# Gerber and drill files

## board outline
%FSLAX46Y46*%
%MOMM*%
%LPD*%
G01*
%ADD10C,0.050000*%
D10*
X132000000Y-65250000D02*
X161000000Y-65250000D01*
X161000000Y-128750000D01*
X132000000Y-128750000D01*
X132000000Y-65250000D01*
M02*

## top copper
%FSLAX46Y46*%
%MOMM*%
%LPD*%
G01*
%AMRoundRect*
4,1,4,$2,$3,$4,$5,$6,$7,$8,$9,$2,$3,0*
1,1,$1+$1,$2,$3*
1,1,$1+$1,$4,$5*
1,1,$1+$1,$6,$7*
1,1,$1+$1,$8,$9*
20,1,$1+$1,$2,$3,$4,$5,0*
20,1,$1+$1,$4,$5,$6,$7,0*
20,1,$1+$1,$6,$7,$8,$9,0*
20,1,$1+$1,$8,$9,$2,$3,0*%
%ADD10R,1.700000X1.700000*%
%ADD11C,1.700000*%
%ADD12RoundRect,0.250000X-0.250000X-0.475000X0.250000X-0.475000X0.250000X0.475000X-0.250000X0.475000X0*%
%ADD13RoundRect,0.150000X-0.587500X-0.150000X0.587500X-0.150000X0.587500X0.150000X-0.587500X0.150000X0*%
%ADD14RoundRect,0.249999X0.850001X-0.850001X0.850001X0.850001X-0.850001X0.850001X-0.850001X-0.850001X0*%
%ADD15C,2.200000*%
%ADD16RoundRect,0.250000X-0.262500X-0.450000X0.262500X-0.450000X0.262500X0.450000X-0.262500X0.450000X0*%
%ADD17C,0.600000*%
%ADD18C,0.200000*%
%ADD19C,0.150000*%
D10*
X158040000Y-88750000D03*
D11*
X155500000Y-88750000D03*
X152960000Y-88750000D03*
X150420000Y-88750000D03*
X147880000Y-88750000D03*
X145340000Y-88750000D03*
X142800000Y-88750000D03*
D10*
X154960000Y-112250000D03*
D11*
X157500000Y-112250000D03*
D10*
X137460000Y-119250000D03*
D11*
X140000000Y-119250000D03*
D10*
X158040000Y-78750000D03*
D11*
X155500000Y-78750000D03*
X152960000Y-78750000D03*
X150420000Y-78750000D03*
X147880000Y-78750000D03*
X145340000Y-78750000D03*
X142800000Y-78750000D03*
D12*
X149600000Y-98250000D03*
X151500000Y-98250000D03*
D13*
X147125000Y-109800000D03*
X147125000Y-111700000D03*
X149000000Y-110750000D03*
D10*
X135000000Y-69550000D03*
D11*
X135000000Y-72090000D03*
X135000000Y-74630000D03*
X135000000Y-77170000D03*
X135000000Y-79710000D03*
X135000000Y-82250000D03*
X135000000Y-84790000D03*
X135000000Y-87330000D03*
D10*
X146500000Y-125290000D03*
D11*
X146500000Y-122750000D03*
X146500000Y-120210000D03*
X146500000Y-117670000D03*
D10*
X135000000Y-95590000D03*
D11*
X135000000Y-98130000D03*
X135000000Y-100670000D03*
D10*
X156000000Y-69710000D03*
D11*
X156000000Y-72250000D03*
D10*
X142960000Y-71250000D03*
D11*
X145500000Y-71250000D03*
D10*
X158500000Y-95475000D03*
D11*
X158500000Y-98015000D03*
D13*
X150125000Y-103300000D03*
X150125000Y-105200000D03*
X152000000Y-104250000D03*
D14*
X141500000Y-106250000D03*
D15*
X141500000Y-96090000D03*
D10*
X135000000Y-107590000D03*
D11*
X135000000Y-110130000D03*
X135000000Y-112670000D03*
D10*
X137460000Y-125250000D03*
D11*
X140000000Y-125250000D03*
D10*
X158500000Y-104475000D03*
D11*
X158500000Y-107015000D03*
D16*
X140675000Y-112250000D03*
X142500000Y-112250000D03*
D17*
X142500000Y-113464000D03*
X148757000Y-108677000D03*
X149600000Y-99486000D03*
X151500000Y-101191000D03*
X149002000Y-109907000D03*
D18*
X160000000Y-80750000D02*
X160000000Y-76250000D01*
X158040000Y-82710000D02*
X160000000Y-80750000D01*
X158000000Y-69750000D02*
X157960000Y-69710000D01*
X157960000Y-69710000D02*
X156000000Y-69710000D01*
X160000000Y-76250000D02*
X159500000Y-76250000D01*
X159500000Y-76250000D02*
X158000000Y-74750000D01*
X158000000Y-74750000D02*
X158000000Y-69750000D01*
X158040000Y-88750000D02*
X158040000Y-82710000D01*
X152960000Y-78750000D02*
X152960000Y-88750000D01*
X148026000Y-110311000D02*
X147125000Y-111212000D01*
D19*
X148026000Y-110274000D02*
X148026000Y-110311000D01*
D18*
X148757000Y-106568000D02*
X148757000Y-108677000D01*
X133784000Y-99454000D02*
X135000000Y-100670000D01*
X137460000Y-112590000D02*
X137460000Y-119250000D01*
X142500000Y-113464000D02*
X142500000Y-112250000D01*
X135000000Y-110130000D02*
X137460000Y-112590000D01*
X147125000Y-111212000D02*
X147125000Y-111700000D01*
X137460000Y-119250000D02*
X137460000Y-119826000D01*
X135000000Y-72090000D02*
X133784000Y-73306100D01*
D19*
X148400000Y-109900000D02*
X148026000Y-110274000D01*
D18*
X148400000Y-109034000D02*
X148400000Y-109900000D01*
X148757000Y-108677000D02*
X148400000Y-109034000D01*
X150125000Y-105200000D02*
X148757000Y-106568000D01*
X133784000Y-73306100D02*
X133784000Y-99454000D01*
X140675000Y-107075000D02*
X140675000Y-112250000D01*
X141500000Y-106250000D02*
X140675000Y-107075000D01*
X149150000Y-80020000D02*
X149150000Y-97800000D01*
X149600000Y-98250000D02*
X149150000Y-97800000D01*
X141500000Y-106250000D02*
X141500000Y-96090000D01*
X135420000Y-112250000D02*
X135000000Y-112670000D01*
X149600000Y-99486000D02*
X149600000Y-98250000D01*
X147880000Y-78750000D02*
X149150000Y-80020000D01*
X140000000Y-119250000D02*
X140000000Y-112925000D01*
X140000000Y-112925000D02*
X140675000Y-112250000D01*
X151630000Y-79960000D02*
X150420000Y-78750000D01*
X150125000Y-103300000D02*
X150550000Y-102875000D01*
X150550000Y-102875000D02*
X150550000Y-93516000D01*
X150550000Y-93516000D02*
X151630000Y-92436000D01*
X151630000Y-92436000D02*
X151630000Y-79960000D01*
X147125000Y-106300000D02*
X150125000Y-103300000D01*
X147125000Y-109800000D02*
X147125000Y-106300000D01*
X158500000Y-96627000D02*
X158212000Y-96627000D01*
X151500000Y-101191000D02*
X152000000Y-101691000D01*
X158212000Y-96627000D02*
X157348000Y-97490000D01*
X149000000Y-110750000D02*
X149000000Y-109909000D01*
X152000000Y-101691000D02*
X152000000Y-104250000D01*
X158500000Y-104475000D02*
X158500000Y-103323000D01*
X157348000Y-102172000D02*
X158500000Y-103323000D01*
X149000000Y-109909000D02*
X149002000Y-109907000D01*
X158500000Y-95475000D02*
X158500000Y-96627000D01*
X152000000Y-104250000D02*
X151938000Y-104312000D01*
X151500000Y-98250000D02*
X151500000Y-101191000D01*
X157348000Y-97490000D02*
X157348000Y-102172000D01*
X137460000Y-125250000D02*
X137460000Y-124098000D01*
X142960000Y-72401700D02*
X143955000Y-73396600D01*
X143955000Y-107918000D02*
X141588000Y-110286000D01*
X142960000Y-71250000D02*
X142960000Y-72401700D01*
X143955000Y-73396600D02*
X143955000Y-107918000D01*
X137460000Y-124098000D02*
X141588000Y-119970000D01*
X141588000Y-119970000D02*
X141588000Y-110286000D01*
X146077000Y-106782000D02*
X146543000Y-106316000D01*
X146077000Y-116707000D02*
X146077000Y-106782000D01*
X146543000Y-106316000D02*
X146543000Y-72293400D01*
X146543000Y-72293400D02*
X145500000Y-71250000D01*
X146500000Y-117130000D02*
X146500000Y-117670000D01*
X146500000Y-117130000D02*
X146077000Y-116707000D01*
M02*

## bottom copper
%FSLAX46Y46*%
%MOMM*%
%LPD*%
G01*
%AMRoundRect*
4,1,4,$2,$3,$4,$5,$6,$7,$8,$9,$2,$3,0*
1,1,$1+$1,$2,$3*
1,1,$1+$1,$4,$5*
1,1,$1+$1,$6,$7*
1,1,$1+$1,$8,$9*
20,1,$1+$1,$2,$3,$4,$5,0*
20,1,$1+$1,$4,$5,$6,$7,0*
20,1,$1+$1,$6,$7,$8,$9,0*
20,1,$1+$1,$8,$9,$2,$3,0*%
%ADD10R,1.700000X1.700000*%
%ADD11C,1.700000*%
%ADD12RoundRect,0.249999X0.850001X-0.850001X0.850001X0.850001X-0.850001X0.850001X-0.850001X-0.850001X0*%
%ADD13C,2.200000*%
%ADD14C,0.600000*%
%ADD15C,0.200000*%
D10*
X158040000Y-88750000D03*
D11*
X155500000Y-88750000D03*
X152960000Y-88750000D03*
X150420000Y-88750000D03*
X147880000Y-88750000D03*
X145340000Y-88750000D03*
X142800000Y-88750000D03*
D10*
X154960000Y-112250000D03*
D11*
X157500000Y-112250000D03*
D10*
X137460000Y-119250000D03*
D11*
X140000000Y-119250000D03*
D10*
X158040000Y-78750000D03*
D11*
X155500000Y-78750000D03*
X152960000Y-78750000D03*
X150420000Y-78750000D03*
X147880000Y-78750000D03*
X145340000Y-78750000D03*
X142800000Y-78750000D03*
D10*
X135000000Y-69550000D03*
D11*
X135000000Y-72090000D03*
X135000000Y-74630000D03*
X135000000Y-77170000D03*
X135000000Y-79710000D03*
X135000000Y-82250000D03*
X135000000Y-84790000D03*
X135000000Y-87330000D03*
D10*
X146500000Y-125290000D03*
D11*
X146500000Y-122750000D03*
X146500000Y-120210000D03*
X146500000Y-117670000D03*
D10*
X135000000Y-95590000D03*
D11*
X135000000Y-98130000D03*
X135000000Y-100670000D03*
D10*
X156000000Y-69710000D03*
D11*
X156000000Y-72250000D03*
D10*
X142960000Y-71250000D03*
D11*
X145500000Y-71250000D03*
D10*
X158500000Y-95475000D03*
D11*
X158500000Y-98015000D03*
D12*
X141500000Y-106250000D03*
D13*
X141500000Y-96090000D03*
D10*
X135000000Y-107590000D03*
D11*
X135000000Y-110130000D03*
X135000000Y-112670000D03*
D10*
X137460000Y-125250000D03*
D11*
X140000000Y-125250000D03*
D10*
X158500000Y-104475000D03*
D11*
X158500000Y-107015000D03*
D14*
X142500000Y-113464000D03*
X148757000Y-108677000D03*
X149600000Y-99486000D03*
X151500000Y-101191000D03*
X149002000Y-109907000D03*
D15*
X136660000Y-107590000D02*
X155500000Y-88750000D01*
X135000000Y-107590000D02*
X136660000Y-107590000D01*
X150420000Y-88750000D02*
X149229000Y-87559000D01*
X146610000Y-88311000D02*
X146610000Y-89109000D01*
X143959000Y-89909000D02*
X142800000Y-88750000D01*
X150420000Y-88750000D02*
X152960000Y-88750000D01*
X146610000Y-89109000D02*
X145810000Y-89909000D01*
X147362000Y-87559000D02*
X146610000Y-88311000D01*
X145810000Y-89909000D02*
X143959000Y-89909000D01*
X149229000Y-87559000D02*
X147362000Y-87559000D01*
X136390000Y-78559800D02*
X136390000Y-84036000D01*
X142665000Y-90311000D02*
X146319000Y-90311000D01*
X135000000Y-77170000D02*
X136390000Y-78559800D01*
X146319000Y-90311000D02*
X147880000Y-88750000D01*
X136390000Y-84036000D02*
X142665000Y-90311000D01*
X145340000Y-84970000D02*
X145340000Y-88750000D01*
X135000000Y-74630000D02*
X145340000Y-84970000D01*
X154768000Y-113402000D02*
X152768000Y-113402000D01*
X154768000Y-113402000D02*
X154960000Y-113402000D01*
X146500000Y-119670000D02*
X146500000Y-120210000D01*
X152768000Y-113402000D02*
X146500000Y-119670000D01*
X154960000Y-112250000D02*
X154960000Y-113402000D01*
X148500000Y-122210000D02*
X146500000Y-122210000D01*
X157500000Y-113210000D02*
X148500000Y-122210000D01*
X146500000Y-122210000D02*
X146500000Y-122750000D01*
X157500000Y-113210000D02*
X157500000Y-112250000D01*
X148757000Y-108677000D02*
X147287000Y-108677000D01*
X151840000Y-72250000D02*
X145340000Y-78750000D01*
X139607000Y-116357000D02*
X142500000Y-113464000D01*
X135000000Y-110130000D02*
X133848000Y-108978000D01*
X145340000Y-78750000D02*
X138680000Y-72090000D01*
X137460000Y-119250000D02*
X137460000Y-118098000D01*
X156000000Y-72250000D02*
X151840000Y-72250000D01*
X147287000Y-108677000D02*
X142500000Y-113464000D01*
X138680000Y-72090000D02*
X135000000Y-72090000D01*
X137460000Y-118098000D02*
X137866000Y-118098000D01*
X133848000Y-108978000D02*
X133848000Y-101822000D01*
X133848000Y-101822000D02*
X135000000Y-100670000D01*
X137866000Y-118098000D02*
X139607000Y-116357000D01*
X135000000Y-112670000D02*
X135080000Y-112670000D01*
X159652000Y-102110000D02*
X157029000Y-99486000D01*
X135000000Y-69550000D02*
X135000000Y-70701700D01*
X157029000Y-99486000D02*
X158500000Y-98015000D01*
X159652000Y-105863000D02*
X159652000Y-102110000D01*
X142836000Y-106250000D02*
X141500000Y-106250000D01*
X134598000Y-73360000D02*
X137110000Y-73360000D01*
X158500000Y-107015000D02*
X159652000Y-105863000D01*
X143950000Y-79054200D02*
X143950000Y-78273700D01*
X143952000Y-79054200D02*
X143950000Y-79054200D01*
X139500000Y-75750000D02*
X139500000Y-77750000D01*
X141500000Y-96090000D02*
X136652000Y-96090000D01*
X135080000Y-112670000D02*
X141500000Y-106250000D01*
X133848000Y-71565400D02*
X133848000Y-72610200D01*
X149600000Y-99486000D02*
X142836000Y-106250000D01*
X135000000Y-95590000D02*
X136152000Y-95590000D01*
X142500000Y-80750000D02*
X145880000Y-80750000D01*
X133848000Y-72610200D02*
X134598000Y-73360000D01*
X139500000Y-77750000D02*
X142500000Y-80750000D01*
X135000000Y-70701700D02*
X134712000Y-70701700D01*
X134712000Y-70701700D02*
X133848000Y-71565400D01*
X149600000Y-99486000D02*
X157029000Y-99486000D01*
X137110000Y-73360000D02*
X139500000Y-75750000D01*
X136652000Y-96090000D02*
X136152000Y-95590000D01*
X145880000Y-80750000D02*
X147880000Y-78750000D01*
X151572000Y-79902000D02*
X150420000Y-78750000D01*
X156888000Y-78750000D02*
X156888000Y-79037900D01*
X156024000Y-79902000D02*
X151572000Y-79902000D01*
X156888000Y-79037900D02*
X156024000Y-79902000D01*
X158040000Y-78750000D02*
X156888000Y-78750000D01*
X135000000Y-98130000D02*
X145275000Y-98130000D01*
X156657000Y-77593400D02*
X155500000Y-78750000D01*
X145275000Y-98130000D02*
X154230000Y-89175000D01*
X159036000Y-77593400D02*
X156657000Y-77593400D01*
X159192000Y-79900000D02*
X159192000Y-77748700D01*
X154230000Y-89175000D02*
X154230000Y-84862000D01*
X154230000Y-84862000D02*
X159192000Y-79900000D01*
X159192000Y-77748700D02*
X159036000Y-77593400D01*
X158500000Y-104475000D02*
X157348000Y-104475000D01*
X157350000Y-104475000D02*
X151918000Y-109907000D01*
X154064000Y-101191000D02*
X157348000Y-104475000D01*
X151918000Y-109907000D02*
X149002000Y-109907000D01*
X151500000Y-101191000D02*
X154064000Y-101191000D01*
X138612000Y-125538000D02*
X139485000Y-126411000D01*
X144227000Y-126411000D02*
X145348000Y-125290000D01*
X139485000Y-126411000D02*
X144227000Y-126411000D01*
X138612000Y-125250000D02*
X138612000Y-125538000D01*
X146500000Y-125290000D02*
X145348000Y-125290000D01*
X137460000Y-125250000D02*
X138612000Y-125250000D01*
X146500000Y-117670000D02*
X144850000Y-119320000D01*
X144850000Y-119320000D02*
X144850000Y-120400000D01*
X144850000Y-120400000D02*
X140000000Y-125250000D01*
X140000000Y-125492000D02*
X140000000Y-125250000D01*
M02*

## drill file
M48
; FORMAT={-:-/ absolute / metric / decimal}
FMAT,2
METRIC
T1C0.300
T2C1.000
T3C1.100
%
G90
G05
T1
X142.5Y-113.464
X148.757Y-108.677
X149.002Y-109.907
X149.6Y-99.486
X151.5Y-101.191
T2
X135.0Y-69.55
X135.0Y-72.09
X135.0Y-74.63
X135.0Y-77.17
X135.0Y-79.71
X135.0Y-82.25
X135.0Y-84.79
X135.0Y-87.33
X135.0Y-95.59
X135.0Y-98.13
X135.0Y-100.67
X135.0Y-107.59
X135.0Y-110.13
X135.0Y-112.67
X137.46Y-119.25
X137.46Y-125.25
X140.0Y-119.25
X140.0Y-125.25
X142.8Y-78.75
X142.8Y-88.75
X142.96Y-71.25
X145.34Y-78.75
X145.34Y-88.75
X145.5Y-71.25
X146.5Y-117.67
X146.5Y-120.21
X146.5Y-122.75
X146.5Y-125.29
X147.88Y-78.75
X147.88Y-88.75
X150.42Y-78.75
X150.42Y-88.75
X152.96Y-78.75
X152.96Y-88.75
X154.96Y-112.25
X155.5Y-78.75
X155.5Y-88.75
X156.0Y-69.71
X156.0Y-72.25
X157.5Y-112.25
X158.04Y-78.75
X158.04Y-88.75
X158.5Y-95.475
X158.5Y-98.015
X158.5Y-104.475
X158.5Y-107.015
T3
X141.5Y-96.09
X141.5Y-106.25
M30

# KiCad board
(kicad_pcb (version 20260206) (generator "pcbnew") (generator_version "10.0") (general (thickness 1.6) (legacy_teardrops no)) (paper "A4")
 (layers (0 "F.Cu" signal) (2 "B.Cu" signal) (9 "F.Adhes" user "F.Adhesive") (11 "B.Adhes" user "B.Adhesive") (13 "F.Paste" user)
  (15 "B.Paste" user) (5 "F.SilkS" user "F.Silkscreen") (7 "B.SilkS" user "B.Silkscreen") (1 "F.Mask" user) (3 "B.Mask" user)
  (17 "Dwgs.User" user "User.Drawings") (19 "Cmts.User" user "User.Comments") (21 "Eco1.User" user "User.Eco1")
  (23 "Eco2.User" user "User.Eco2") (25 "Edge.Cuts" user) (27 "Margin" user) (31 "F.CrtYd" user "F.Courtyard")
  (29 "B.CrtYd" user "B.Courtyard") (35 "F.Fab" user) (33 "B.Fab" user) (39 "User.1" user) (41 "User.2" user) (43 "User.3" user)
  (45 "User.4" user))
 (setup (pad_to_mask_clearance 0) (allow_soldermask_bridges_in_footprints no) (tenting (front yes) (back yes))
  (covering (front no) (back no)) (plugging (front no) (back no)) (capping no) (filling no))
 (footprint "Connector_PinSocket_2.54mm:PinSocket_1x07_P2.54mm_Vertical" (layer "F.Cu") (at 158.04 88.75 -90)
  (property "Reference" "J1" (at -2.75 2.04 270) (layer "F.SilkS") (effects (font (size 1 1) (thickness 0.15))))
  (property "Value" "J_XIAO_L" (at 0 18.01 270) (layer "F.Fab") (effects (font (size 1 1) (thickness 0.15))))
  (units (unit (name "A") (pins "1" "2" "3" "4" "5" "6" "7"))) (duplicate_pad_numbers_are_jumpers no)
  (pad "1" thru_hole rect (at 0 0 270) (size 1.7 1.7) (drill 1) (layers "*.Cu" "*.Mask") (remove_unused_layers no) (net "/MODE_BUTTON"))
  (pad "2" thru_hole circle (at 0 2.54 270) (size 1.7 1.7) (drill 1) (layers "*.Cu" "*.Mask") (remove_unused_layers no) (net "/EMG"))
  (pad "3" thru_hole circle (at 0 5.08 270) (size 1.7 1.7) (drill 1) (layers "*.Cu" "*.Mask") (remove_unused_layers no) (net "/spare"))
  (pad "4" thru_hole circle (at 0 7.62 270) (size 1.7 1.7) (drill 1) (layers "*.Cu" "*.Mask") (remove_unused_layers no) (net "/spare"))
  (pad "5" thru_hole circle (at 0 10.16 270) (size 1.7 1.7) (drill 1) (layers "*.Cu" "*.Mask") (remove_unused_layers no) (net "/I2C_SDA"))
  (pad "6" thru_hole circle (at 0 12.7 270) (size 1.7 1.7) (drill 1) (layers "*.Cu" "*.Mask") (remove_unused_layers no) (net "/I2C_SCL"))
  (pad "7" thru_hole circle (at 0 15.24 270) (size 1.7 1.7) (drill 1) (layers "*.Cu" "*.Mask") (remove_unused_layers no) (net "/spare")))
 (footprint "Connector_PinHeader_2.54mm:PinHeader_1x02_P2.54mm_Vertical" (layer "F.Cu") (at 154.96 112.25 90)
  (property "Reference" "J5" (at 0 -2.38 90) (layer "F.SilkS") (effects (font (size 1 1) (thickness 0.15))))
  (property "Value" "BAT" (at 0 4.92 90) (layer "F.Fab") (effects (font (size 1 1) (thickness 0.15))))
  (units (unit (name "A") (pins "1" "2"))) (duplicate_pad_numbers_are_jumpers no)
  (pad "1" thru_hole rect (at 0 0 90) (size 1.7 1.7) (drill 1) (layers "*.Cu" "*.Mask") (remove_unused_layers no) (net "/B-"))
  (pad "2" thru_hole circle (at 0 2.54 90) (size 1.7 1.7) (drill 1) (layers "*.Cu" "*.Mask") (remove_unused_layers no) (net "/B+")))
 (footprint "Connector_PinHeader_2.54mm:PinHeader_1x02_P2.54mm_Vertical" (layer "F.Cu") (at 137.46 119.25 90)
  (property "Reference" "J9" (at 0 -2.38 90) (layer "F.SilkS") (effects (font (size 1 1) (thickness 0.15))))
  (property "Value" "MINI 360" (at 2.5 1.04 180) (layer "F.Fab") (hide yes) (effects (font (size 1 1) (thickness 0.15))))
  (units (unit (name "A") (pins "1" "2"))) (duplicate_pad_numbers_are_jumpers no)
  (pad "1" thru_hole rect (at 0 0 90) (size 1.7 1.7) (drill 1) (layers "*.Cu" "*.Mask") (remove_unused_layers no) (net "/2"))
  (pad "2" thru_hole circle (at 0 2.54 90) (size 1.7 1.7) (drill 1) (layers "*.Cu" "*.Mask") (remove_unused_layers no) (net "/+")))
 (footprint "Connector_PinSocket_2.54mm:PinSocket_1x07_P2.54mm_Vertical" (layer "F.Cu") (at 158.04 78.75 -90)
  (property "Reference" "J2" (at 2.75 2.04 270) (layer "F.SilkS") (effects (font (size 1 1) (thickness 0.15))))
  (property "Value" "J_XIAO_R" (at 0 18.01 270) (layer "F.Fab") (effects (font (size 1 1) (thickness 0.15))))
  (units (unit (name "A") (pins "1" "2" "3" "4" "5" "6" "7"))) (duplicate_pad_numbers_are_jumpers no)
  (pad "1" thru_hole rect (at 0 0 270) (size 1.7 1.7) (drill 1) (layers "*.Cu" "*.Mask") (remove_unused_layers no) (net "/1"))
  (pad "2" thru_hole circle (at 0 2.54 270) (size 1.7 1.7) (drill 1) (layers "*.Cu" "*.Mask") (remove_unused_layers no) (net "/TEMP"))
  (pad "3" thru_hole circle (at 0 5.08 270) (size 1.7 1.7) (drill 1) (layers "*.Cu" "*.Mask") (remove_unused_layers no) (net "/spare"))
  (pad "4" thru_hole circle (at 0 7.62 270) (size 1.7 1.7) (drill 1) (layers "*.Cu" "*.Mask") (remove_unused_layers no) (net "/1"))
  (pad "5" thru_hole circle (at 0 10.16 270) (size 1.7 1.7) (drill 1) (layers "*.Cu" "*.Mask") (remove_unused_layers no) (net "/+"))
  (pad "6" thru_hole circle (at 0 12.7 270) (size 1.7 1.7) (drill 1) (layers "*.Cu" "*.Mask") (remove_unused_layers no) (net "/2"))
  (pad "7" thru_hole circle (at 0 15.24 270) (size 1.7 1.7) (drill 1) (layers "*.Cu" "*.Mask") (remove_unused_layers no) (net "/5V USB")))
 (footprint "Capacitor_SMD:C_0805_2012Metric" (layer "F.Cu") (at 150.55 98.25)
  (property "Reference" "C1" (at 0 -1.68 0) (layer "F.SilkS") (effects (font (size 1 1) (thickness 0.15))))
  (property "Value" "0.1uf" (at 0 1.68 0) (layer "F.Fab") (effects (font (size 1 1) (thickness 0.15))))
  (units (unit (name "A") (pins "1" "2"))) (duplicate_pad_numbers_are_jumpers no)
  (pad "1" smd roundrect (at -0.95 0) (size 1 1.45) (layers "F.Cu" "F.Mask" "F.Paste") (roundrect_rratio 0.25) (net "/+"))
  (pad "2" smd roundrect (at 0.95 0) (size 1 1.45) (layers "F.Cu" "F.Mask" "F.Paste") (roundrect_rratio 0.25) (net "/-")))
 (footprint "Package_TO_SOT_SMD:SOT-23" (layer "F.Cu") (at 148.0625 110.75)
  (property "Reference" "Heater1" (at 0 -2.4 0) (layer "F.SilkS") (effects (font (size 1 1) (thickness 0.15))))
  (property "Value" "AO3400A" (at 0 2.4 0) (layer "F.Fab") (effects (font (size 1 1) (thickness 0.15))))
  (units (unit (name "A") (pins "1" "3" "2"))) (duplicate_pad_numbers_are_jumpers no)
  (pad "1" smd roundrect (at -0.9375 -0.95) (size 1.475 0.6) (layers "F.Cu" "F.Mask" "F.Paste") (roundrect_rratio 0.25) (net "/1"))
  (pad "2" smd roundrect (at -0.9375 0.95) (size 1.475 0.6) (layers "F.Cu" "F.Mask" "F.Paste") (roundrect_rratio 0.25) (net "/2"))
  (pad "3" smd roundrect (at 0.9375 0) (size 1.475 0.6) (layers "F.Cu" "F.Mask" "F.Paste") (roundrect_rratio 0.25) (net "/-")))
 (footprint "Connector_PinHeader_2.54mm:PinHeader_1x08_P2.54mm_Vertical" (layer "F.Cu") (at 135 69.55)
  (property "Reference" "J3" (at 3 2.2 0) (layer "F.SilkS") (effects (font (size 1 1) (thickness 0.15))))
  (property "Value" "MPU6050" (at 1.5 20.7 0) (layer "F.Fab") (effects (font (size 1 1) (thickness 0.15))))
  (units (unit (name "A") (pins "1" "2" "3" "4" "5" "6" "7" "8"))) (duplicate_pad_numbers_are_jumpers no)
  (pad "1" thru_hole rect (at 0 0) (size 1.7 1.7) (drill 1) (layers "*.Cu" "*.Mask") (remove_unused_layers no) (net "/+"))
  (pad "2" thru_hole circle (at 0 2.54) (size 1.7 1.7) (drill 1) (layers "*.Cu" "*.Mask") (remove_unused_layers no) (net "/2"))
  (pad "3" thru_hole circle (at 0 5.08) (size 1.7 1.7) (drill 1) (layers "*.Cu" "*.Mask") (remove_unused_layers no) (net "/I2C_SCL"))
  (pad "4" thru_hole circle (at 0 7.62) (size 1.7 1.7) (drill 1) (layers "*.Cu" "*.Mask") (remove_unused_layers no) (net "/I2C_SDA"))
  (pad "5" thru_hole circle (at 0 10.16) (size 1.7 1.7) (drill 1) (layers "*.Cu" "*.Mask") (remove_unused_layers no) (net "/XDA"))
  (pad "6" thru_hole circle (at 0 12.7) (size 1.7 1.7) (drill 1) (layers "*.Cu" "*.Mask") (remove_unused_layers no) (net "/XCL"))
  (pad "7" thru_hole circle (at 0 15.24) (size 1.7 1.7) (drill 1) (layers "*.Cu" "*.Mask") (remove_unused_layers no) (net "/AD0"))
  (pad "8" thru_hole circle (at 0 17.78) (size 1.7 1.7) (drill 1) (layers "*.Cu" "*.Mask") (remove_unused_layers no) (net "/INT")))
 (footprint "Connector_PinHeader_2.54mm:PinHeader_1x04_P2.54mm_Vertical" (layer "F.Cu") (at 146.5 125.29 180)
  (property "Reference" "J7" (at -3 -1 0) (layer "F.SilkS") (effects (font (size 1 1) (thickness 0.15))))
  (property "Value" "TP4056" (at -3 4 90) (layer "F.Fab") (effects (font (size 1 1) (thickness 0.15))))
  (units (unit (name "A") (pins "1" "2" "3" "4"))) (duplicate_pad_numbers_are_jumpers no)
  (pad "1" thru_hole rect (at 0 0 180) (size 1.7 1.7) (drill 1) (layers "*.Cu" "*.Mask") (remove_unused_layers no) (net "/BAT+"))
  (pad "2" thru_hole circle (at 0 2.54 180) (size 1.7 1.7) (drill 1) (layers "*.Cu" "*.Mask") (remove_unused_layers no) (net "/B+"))
  (pad "3" thru_hole circle (at 0 5.08 180) (size 1.7 1.7) (drill 1) (layers "*.Cu" "*.Mask") (remove_unused_layers no) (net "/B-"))
  (pad "4" thru_hole circle (at 0 7.62 180) (size 1.7 1.7) (drill 1) (layers "*.Cu" "*.Mask") (remove_unused_layers no) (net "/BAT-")))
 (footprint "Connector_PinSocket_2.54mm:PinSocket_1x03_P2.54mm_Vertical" (layer "F.Cu") (at 135 95.59)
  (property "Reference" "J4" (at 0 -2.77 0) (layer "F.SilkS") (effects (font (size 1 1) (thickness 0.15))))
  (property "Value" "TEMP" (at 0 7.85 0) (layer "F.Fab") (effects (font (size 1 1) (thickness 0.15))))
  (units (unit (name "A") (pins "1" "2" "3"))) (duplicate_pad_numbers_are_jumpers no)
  (pad "1" thru_hole rect (at 0 0) (size 1.7 1.7) (drill 1) (layers "*.Cu" "*.Mask") (remove_unused_layers no) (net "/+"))
  (pad "2" thru_hole circle (at 0 2.54) (size 1.7 1.7) (drill 1) (layers "*.Cu" "*.Mask") (remove_unused_layers no) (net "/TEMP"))
  (pad "3" thru_hole circle (at 0 5.08) (size 1.7 1.7) (drill 1) (layers "*.Cu" "*.Mask") (remove_unused_layers no) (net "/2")))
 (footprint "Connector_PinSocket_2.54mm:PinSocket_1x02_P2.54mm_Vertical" (layer "F.Cu") (at 156 69.71)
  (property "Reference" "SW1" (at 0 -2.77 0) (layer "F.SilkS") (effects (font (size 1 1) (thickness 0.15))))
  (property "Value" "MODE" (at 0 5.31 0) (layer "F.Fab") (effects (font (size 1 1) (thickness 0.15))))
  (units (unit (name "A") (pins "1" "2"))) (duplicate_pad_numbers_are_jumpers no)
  (pad "1" thru_hole rect (at 0 0) (size 1.7 1.7) (drill 1) (layers "*.Cu" "*.Mask") (remove_unused_layers no) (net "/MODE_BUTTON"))
  (pad "2" thru_hole circle (at 0 2.54) (size 1.7 1.7) (drill 1) (layers "*.Cu" "*.Mask") (remove_unused_layers no) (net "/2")))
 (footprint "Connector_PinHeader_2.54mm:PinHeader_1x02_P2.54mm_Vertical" (layer "F.Cu") (at 142.96 71.25 90)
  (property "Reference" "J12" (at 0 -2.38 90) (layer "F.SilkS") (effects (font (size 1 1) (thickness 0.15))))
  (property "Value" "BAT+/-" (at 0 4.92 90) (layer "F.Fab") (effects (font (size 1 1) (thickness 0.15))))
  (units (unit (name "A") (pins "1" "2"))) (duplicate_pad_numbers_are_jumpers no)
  (pad "1" thru_hole rect (at 0 0 90) (size 1.7 1.7) (drill 1) (layers "*.Cu" "*.Mask") (remove_unused_layers no) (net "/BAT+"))
  (pad "2" thru_hole circle (at 0 2.54 90) (size 1.7 1.7) (drill 1) (layers "*.Cu" "*.Mask") (remove_unused_layers no) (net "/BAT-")))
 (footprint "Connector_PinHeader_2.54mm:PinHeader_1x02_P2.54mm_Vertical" (layer "F.Cu") (at 158.5 95.475)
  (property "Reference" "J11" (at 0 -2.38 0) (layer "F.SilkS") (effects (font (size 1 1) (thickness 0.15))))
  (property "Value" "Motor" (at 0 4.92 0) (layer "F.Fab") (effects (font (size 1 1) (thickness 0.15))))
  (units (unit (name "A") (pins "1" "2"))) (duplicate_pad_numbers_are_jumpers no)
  (pad "1" thru_hole rect (at 0 0) (size 1.7 1.7) (drill 1) (layers "*.Cu" "*.Mask") (remove_unused_layers no) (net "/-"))
  (pad "2" thru_hole circle (at 0 2.54) (size 1.7 1.7) (drill 1) (layers "*.Cu" "*.Mask") (remove_unused_layers no) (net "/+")))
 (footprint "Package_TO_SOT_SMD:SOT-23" (layer "F.Cu") (at 151.0625 104.25)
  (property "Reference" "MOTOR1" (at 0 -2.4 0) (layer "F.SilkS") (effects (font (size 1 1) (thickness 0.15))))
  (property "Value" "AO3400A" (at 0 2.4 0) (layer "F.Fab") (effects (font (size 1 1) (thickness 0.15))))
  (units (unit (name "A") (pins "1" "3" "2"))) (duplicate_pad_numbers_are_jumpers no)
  (pad "1" smd roundrect (at -0.9375 -0.95) (size 1.475 0.6) (layers "F.Cu" "F.Mask" "F.Paste") (roundrect_rratio 0.25) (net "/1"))
  (pad "2" smd roundrect (at -0.9375 0.95) (size 1.475 0.6) (layers "F.Cu" "F.Mask" "F.Paste") (roundrect_rratio 0.25) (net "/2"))
  (pad "3" smd roundrect (at 0.9375 0) (size 1.475 0.6) (layers "F.Cu" "F.Mask" "F.Paste") (roundrect_rratio 0.25) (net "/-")))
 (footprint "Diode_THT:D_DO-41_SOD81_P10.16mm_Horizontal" (layer "F.Cu") (at 141.5 106.25 90)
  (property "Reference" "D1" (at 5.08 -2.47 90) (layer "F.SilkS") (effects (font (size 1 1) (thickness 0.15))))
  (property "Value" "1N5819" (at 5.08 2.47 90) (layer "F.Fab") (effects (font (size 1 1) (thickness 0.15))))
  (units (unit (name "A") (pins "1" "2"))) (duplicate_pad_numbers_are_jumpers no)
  (pad "1" thru_hole roundrect (at 0 0 90) (size 2.2 2.2) (drill 1.1) (layers "*.Cu" "*.Mask") (remove_unused_layers no)
   (roundrect_rratio 0.113636) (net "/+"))
  (pad "2" thru_hole circle (at 10.16 0 90) (size 2.2 2.2) (drill 1.1) (layers "*.Cu" "*.Mask") (remove_unused_layers no) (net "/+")))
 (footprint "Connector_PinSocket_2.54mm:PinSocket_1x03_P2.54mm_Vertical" (layer "F.Cu") (at 135 107.59)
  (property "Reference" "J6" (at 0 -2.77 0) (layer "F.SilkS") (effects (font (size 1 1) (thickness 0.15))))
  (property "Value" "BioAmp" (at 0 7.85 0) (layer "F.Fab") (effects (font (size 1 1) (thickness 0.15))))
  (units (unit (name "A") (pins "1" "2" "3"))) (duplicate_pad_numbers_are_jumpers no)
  (pad "1" thru_hole rect (at 0 0) (size 1.7 1.7) (drill 1) (layers "*.Cu" "*.Mask") (remove_unused_layers no) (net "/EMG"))
  (pad "2" thru_hole circle (at 0 2.54) (size 1.7 1.7) (drill 1) (layers "*.Cu" "*.Mask") (remove_unused_layers no) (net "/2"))
  (pad "3" thru_hole circle (at 0 5.08) (size 1.7 1.7) (drill 1) (layers "*.Cu" "*.Mask") (remove_unused_layers no) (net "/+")))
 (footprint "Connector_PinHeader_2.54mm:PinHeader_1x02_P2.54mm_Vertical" (layer "F.Cu") (at 137.46 125.25 90)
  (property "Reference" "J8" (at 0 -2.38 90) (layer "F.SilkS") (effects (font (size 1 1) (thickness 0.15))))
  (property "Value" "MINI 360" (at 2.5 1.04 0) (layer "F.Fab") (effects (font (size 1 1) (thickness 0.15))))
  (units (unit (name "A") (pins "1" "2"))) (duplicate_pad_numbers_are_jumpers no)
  (pad "1" thru_hole rect (at 0 0 90) (size 1.7 1.7) (drill 1) (layers "*.Cu" "*.Mask") (remove_unused_layers no) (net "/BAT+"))
  (pad "2" thru_hole circle (at 0 2.54 90) (size 1.7 1.7) (drill 1) (layers "*.Cu" "*.Mask") (remove_unused_layers no) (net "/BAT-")))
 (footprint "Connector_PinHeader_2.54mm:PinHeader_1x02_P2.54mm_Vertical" (layer "F.Cu") (at 158.5 104.475)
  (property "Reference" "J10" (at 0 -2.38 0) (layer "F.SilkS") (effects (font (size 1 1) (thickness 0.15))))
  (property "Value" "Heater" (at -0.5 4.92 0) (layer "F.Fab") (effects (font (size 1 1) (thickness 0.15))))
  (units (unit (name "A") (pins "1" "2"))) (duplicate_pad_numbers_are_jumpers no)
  (pad "1" thru_hole rect (at 0 0) (size 1.7 1.7) (drill 1) (layers "*.Cu" "*.Mask") (remove_unused_layers no) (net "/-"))
  (pad "2" thru_hole circle (at 0 2.54) (size 1.7 1.7) (drill 1) (layers "*.Cu" "*.Mask") (remove_unused_layers no) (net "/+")))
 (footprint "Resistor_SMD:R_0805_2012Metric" (layer "F.Cu") (at 141.5875 112.25)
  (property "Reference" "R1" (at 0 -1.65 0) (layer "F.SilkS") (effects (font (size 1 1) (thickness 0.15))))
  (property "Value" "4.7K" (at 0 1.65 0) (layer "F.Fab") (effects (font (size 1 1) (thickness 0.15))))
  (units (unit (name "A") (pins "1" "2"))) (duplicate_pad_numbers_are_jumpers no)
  (pad "1" smd roundrect (at -0.9125 0) (size 1.025 1.4) (layers "F.Cu" "F.Mask" "F.Paste") (roundrect_rratio 0.243902) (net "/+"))
  (pad "2" smd roundrect (at 0.9125 0) (size 1.025 1.4) (layers "F.Cu" "F.Mask" "F.Paste") (roundrect_rratio 0.243902) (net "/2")))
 (gr_rect (start 132 65.25) (end 161 128.75) (stroke (width 0.05) (type default)) (fill no) (layer "Edge.Cuts"))
 (segment (start 160 80.75) (end 160 76.25) (width 0.2) (layer "F.Cu") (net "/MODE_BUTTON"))
 (segment (start 158.04 82.71) (end 160 80.75) (width 0.2) (layer "F.Cu") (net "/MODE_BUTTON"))
 (segment (start 158 69.75) (end 157.96 69.71) (width 0.2) (layer "F.Cu") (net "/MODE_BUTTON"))
 (segment (start 157.96 69.71) (end 156 69.71) (width 0.2) (layer "F.Cu") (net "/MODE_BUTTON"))
 (segment (start 160 76.25) (end 159.5 76.25) (width 0.2) (layer "F.Cu") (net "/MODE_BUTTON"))
 (segment (start 159.5 76.25) (end 158 74.75) (width 0.2) (layer "F.Cu") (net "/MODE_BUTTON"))
 (segment (start 158 74.75) (end 158 69.75) (width 0.2) (layer "F.Cu") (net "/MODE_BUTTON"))
 (segment (start 158.04 88.75) (end 158.04 82.71) (width 0.2) (layer "F.Cu") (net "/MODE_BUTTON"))
 (segment (start 136.66 107.59) (end 155.5 88.75) (width 0.2) (layer "B.Cu") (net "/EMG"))
 (segment (start 135 107.59) (end 136.66 107.59) (width 0.2) (layer "B.Cu") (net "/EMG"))
 (segment (start 152.96 78.75) (end 152.96 88.75) (width 0.2) (layer "F.Cu") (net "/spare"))
 (segment (start 150.42 88.75) (end 149.229 87.559) (width 0.2) (layer "B.Cu") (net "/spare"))
 (segment (start 146.61 88.311) (end 146.61 89.109) (width 0.2) (layer "B.Cu") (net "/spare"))
 (segment (start 143.959 89.909) (end 142.8 88.75) (width 0.2) (layer "B.Cu") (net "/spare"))
 (segment (start 150.42 88.75) (end 152.96 88.75) (width 0.2) (layer "B.Cu") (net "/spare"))
 (segment (start 146.61 89.109) (end 145.81 89.909) (width 0.2) (layer "B.Cu") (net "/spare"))
 (segment (start 147.362 87.559) (end 146.61 88.311) (width 0.2) (layer "B.Cu") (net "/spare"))
 (segment (start 145.81 89.909) (end 143.959 89.909) (width 0.2) (layer "B.Cu") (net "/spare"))
 (segment (start 149.229 87.559) (end 147.362 87.559) (width 0.2) (layer "B.Cu") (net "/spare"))
 (segment (start 136.39 78.5598) (end 136.39 84.036) (width 0.2) (layer "B.Cu") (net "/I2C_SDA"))
 (segment (start 142.665 90.311) (end 146.319 90.311) (width 0.2) (layer "B.Cu") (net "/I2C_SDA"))
 (segment (start 135 77.17) (end 136.39 78.5598) (width 0.2) (layer "B.Cu") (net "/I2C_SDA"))
 (segment (start 146.319 90.311) (end 147.88 88.75) (width 0.2) (layer "B.Cu") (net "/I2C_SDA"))
 (segment (start 136.39 84.036) (end 142.665 90.311) (width 0.2) (layer "B.Cu") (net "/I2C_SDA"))
 (segment (start 145.34 84.97) (end 145.34 88.75) (width 0.2) (layer "B.Cu") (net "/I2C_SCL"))
 (segment (start 135 74.63) (end 145.34 84.97) (width 0.2) (layer "B.Cu") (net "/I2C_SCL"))
 (segment (start 154.768 113.402) (end 152.768 113.402) (width 0.2) (layer "B.Cu") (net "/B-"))
 (segment (start 154.768 113.402) (end 154.96 113.402) (width 0.2) (layer "B.Cu") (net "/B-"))
 (segment (start 146.5 119.67) (end 146.5 120.21) (width 0.2) (layer "B.Cu") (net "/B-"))
 (segment (start 152.768 113.402) (end 146.5 119.67) (width 0.2) (layer "B.Cu") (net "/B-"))
 (segment (start 154.96 112.25) (end 154.96 113.402) (width 0.2) (layer "B.Cu") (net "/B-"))
 (segment (start 148.5 122.21) (end 146.5 122.21) (width 0.2) (layer "B.Cu") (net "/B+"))
 (segment (start 157.5 113.21) (end 148.5 122.21) (width 0.2) (layer "B.Cu") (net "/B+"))
 (segment (start 146.5 122.21) (end 146.5 122.75) (width 0.2) (layer "B.Cu") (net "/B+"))
 (segment (start 157.5 113.21) (end 157.5 112.25) (width 0.2) (layer "B.Cu") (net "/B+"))
 (segment (start 148.026 110.311) (end 147.125 111.212) (width 0.2) (layer "F.Cu") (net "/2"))
 (segment (start 148.026 110.274) (end 148.026 110.311) (width 0.15) (layer "F.Cu") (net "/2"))
 (segment (start 148.757 106.568) (end 148.757 108.677) (width 0.2) (layer "F.Cu") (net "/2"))
 (segment (start 133.784 99.454) (end 135 100.67) (width 0.2) (layer "F.Cu") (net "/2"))
 (segment (start 137.46 112.59) (end 137.46 119.25) (width 0.2) (layer "F.Cu") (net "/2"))
 (segment (start 142.5 113.464) (end 142.5 112.25) (width 0.2) (layer "F.Cu") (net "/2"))
 (segment (start 135 110.13) (end 137.46 112.59) (width 0.2) (layer "F.Cu") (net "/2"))
 (segment (start 147.125 111.212) (end 147.125 111.7) (width 0.2) (layer "F.Cu") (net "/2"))
 (segment (start 137.46 119.25) (end 137.46 119.826) (width 0.2) (layer "F.Cu") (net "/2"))
 (segment (start 135 72.09) (end 133.784 73.3061) (width 0.2) (layer "F.Cu") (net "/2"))
 (segment (start 148.4 109.9) (end 148.026 110.274) (width 0.15) (layer "F.Cu") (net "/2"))
 (segment (start 148.4 109.034) (end 148.4 109.9) (width 0.2) (layer "F.Cu") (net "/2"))
 (segment (start 148.757 108.677) (end 148.4 109.034) (width 0.2) (layer "F.Cu") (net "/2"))
 (segment (start 150.125 105.2) (end 148.757 106.568) (width 0.2) (layer "F.Cu") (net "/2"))
 (segment (start 133.784 73.3061) (end 133.784 99.454) (width 0.2) (layer "F.Cu") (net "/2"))
 (via (at 142.5 113.464) (size 0.6) (drill 0.3) (layers "F.Cu" "B.Cu") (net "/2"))
 (via (at 148.757 108.677) (size 0.6) (drill 0.3) (layers "F.Cu" "B.Cu") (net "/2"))
 (segment (start 148.757 108.677) (end 147.287 108.677) (width 0.2) (layer "B.Cu") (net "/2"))
 (segment (start 151.84 72.25) (end 145.34 78.75) (width 0.2) (layer "B.Cu") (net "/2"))
 (segment (start 139.607 116.357) (end 142.5 113.464) (width 0.2) (layer "B.Cu") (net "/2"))
 (segment (start 135 110.13) (end 133.848 108.978) (width 0.2) (layer "B.Cu") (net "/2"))
 (segment (start 145.34 78.75) (end 138.68 72.09) (width 0.2) (layer "B.Cu") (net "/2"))
 (segment (start 137.46 119.25) (end 137.46 118.098) (width 0.2) (layer "B.Cu") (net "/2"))
 (segment (start 156 72.25) (end 151.84 72.25) (width 0.2) (layer "B.Cu") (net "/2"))
 (segment (start 147.287 108.677) (end 142.5 113.464) (width 0.2) (layer "B.Cu") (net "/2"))
 (segment (start 138.68 72.09) (end 135 72.09) (width 0.2) (layer "B.Cu") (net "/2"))
 (segment (start 137.46 118.098) (end 137.866 118.098) (width 0.2) (layer "B.Cu") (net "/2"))
 (segment (start 133.848 108.978) (end 133.848 101.822) (width 0.2) (layer "B.Cu") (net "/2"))
 (segment (start 133.848 101.822) (end 135 100.67) (width 0.2) (layer "B.Cu") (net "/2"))
 (segment (start 137.866 118.098) (end 139.607 116.357) (width 0.2) (layer "B.Cu") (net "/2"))
 (segment (start 140.675 107.075) (end 140.675 112.25) (width 0.2) (layer "F.Cu") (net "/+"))
 (segment (start 141.5 106.25) (end 140.675 107.075) (width 0.2) (layer "F.Cu") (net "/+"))
 (segment (start 149.15 80.02) (end 149.15 97.8) (width 0.2) (layer "F.Cu") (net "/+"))
 (segment (start 149.6 98.25) (end 149.15 97.8) (width 0.2) (layer "F.Cu") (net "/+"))
 (segment (start 141.5 106.25) (end 141.5 96.09) (width 0.2) (layer "F.Cu") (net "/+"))
 (segment (start 135.42 112.25) (end 135 112.67) (width 0.2) (layer "F.Cu") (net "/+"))
 (segment (start 149.6 99.486) (end 149.6 98.25) (width 0.2) (layer "F.Cu") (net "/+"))
 (segment (start 147.88 78.75) (end 149.15 80.02) (width 0.2) (layer "F.Cu") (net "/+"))
 (segment (start 140 119.25) (end 140 112.925) (width 0.2) (layer "F.Cu") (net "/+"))
 (segment (start 140 112.925) (end 140.675 112.25) (width 0.2) (layer "F.Cu") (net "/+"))
 (via (at 149.6 99.486) (size 0.6) (drill 0.3) (layers "F.Cu" "B.Cu") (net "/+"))
 (segment (start 135 112.67) (end 135.08 112.67) (width 0.2) (layer "B.Cu") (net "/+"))
 (segment (start 159.652 102.11) (end 157.029 99.486) (width 0.2) (layer "B.Cu") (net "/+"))
 (segment (start 135 69.55) (end 135 70.7017) (width 0.2) (layer "B.Cu") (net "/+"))
 (segment (start 157.029 99.486) (end 158.5 98.015) (width 0.2) (layer "B.Cu") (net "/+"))
 (segment (start 159.652 105.863) (end 159.652 102.11) (width 0.2) (layer "B.Cu") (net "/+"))
 (segment (start 142.836 106.25) (end 141.5 106.25) (width 0.2) (layer "B.Cu") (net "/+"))
 (segment (start 134.598 73.36) (end 137.11 73.36) (width 0.2) (layer "B.Cu") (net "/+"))
 (segment (start 158.5 107.015) (end 159.652 105.863) (width 0.2) (layer "B.Cu") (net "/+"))
 (segment (start 143.95 79.0542) (end 143.95 78.2737) (width 0.2) (layer "B.Cu") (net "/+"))
 (segment (start 143.952 79.0542) (end 143.95 79.0542) (width 0.2) (layer "B.Cu") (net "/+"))
 (segment (start 139.5 75.75) (end 139.5 77.75) (width 0.2) (layer "B.Cu") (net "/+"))
 (segment (start 141.5 96.09) (end 136.652 96.09) (width 0.2) (layer "B.Cu") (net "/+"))
 (segment (start 135.08 112.67) (end 141.5 106.25) (width 0.2) (layer "B.Cu") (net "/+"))
 (segment (start 133.848 71.5654) (end 133.848 72.6102) (width 0.2) (layer "B.Cu") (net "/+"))
 (segment (start 149.6 99.486) (end 142.836 106.25) (width 0.2) (layer "B.Cu") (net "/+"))
 (segment (start 135 95.59) (end 136.152 95.59) (width 0.2) (layer "B.Cu") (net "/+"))
 (segment (start 142.5 80.75) (end 145.88 80.75) (width 0.2) (layer "B.Cu") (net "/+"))
 (segment (start 133.848 72.6102) (end 134.598 73.36) (width 0.2) (layer "B.Cu") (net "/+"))
 (segment (start 139.5 77.75) (end 142.5 80.75) (width 0.2) (layer "B.Cu") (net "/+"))
 (segment (start 135 70.7017) (end 134.712 70.7017) (width 0.2) (layer "B.Cu") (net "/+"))
 (segment (start 134.712 70.7017) (end 133.848 71.5654) (width 0.2) (layer "B.Cu") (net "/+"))
 (segment (start 149.6 99.486) (end 157.029 99.486) (width 0.2) (layer "B.Cu") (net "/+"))
 (segment (start 137.11 73.36) (end 139.5 75.75) (width 0.2) (layer "B.Cu") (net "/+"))
 (segment (start 136.652 96.09) (end 136.152 95.59) (width 0.2) (layer "B.Cu") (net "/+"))
 (segment (start 145.88 80.75) (end 147.88 78.75) (width 0.2) (layer "B.Cu") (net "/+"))
 (segment (start 151.63 79.96) (end 150.42 78.75) (width 0.2) (layer "F.Cu") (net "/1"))
 (segment (start 150.125 103.3) (end 150.55 102.875) (width 0.2) (layer "F.Cu") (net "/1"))
 (segment (start 150.55 102.875) (end 150.55 93.516) (width 0.2) (layer "F.Cu") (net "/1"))
 (segment (start 150.55 93.516) (end 151.63 92.436) (width 0.2) (layer "F.Cu") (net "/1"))
 (segment (start 151.63 92.436) (end 151.63 79.96) (width 0.2) (layer "F.Cu") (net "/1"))
 (segment (start 147.125 106.3) (end 150.125 103.3) (width 0.2) (layer "F.Cu") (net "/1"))
 (segment (start 147.125 109.8) (end 147.125 106.3) (width 0.2) (layer "F.Cu") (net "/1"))
 (segment (start 151.572 79.902) (end 150.42 78.75) (width 0.2) (layer "B.Cu") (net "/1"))
 (segment (start 156.888 78.75) (end 156.888 79.0379) (width 0.2) (layer "B.Cu") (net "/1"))
 (segment (start 156.024 79.902) (end 151.572 79.902) (width 0.2) (layer "B.Cu") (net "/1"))
 (segment (start 156.888 79.0379) (end 156.024 79.902) (width 0.2) (layer "B.Cu") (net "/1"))
 (segment (start 158.04 78.75) (end 156.888 78.75) (width 0.2) (layer "B.Cu") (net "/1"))
 (segment (start 135 98.13) (end 145.275 98.13) (width 0.2) (layer "B.Cu") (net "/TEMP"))
 (segment (start 156.657 77.5934) (end 155.5 78.75) (width 0.2) (layer "B.Cu") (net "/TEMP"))
 (segment (start 145.275 98.13) (end 154.23 89.175) (width 0.2) (layer "B.Cu") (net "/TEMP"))
 (segment (start 159.036 77.5934) (end 156.657 77.5934) (width 0.2) (layer "B.Cu") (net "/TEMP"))
 (segment (start 159.192 79.9) (end 159.192 77.7487) (width 0.2) (layer "B.Cu") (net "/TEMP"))
 (segment (start 154.23 89.175) (end 154.23 84.862) (width 0.2) (layer "B.Cu") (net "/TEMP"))
 (segment (start 154.23 84.862) (end 159.192 79.9) (width 0.2) (layer "B.Cu") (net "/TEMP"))
 (segment (start 159.192 77.7487) (end 159.036 77.5934) (width 0.2) (layer "B.Cu") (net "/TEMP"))
 (segment (start 158.5 96.627) (end 158.212 96.627) (width 0.2) (layer "F.Cu") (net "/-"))
 (segment (start 151.5 101.191) (end 152 101.691) (width 0.2) (layer "F.Cu") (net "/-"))
 (segment (start 158.212 96.627) (end 157.348 97.49) (width 0.2) (layer "F.Cu") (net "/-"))
 (segment (start 149 110.75) (end 149 109.909) (width 0.2) (layer "F.Cu") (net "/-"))
 (segment (start 152 101.691) (end 152 104.25) (width 0.2) (layer "F.Cu") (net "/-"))
 (segment (start 158.5 104.475) (end 158.5 103.323) (width 0.2) (layer "F.Cu") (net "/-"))
 (segment (start 157.348 102.172) (end 158.5 103.323) (width 0.2) (layer "F.Cu") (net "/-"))
 (segment (start 149 109.909) (end 149.002 109.907) (width 0.2) (layer "F.Cu") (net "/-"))
 (segment (start 158.5 95.475) (end 158.5 96.627) (width 0.2) (layer "F.Cu") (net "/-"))
 (segment (start 152 104.25) (end 151.938 104.312) (width 0.2) (layer "F.Cu") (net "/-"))
 (segment (start 151.5 98.25) (end 151.5 101.191) (width 0.2) (layer "F.Cu") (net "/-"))
 (segment (start 157.348 97.49) (end 157.348 102.172) (width 0.2) (layer "F.Cu") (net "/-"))
 (via (at 151.5 101.191) (size 0.6) (drill 0.3) (layers "F.Cu" "B.Cu") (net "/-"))
 (via (at 149.002 109.907) (size 0.6) (drill 0.3) (layers "F.Cu" "B.Cu") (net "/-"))
 (segment (start 158.5 104.475) (end 157.348 104.475) (width 0.2) (layer "B.Cu") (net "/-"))
 (segment (start 157.35 104.475) (end 151.918 109.907) (width 0.2) (layer "B.Cu") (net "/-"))
 (segment (start 154.064 101.191) (end 157.348 104.475) (width 0.2) (layer "B.Cu") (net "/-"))
 (segment (start 151.918 109.907) (end 149.002 109.907) (width 0.2) (layer "B.Cu") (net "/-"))
 (segment (start 151.5 101.191) (end 154.064 101.191) (width 0.2) (layer "B.Cu") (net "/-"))
 (segment (start 137.46 125.25) (end 137.46 124.098) (width 0.2) (layer "F.Cu") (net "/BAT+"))
 (segment (start 142.96 72.4017) (end 143.955 73.3966) (width 0.2) (layer "F.Cu") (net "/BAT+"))
 (segment (start 143.955 107.918) (end 141.588 110.286) (width 0.2) (layer "F.Cu") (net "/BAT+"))
 (segment (start 142.96 71.25) (end 142.96 72.4017) (width 0.2) (layer "F.Cu") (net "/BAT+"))
 (segment (start 143.955 73.3966) (end 143.955 107.918) (width 0.2) (layer "F.Cu") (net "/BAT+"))
 (segment (start 137.46 124.098) (end 141.588 119.97) (width 0.2) (layer "F.Cu") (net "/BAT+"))
 (segment (start 141.588 119.97) (end 141.588 110.286) (width 0.2) (layer "F.Cu") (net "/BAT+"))
 (segment (start 138.612 125.538) (end 139.485 126.411) (width 0.2) (layer "B.Cu") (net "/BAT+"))
 (segment (start 144.227 126.411) (end 145.348 125.29) (width 0.2) (layer "B.Cu") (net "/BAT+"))
 (segment (start 139.485 126.411) (end 144.227 126.411) (width 0.2) (layer "B.Cu") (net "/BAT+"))
 (segment (start 138.612 125.25) (end 138.612 125.538) (width 0.2) (layer "B.Cu") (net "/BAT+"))
 (segment (start 146.5 125.29) (end 145.348 125.29) (width 0.2) (layer "B.Cu") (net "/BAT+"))
 (segment (start 137.46 125.25) (end 138.612 125.25) (width 0.2) (layer "B.Cu") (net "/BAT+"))
 (segment (start 146.077 106.782) (end 146.543 106.316) (width 0.2) (layer "F.Cu") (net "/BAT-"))
 (segment (start 146.077 116.707) (end 146.077 106.782) (width 0.2) (layer "F.Cu") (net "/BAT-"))
 (segment (start 146.543 106.316) (end 146.543 72.2934) (width 0.2) (layer "F.Cu") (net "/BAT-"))
 (segment (start 146.543 72.2934) (end 145.5 71.25) (width 0.2) (layer "F.Cu") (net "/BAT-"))
 (segment (start 146.5 117.13) (end 146.5 117.67) (width 0.2) (layer "F.Cu") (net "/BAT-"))
 (segment (start 146.5 117.13) (end 146.077 116.707) (width 0.2) (layer "F.Cu") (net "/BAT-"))
 (segment (start 146.5 117.67) (end 144.85 119.32) (width 0.2) (layer "B.Cu") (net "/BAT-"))
 (segment (start 144.85 119.32) (end 144.85 120.4) (width 0.2) (layer "B.Cu") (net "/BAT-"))
 (segment (start 144.85 120.4) (end 140 125.25) (width 0.2) (layer "B.Cu") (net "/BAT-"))
 (segment (start 140 125.492) (end 140 125.25) (width 0.2) (layer "B.Cu") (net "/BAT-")))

